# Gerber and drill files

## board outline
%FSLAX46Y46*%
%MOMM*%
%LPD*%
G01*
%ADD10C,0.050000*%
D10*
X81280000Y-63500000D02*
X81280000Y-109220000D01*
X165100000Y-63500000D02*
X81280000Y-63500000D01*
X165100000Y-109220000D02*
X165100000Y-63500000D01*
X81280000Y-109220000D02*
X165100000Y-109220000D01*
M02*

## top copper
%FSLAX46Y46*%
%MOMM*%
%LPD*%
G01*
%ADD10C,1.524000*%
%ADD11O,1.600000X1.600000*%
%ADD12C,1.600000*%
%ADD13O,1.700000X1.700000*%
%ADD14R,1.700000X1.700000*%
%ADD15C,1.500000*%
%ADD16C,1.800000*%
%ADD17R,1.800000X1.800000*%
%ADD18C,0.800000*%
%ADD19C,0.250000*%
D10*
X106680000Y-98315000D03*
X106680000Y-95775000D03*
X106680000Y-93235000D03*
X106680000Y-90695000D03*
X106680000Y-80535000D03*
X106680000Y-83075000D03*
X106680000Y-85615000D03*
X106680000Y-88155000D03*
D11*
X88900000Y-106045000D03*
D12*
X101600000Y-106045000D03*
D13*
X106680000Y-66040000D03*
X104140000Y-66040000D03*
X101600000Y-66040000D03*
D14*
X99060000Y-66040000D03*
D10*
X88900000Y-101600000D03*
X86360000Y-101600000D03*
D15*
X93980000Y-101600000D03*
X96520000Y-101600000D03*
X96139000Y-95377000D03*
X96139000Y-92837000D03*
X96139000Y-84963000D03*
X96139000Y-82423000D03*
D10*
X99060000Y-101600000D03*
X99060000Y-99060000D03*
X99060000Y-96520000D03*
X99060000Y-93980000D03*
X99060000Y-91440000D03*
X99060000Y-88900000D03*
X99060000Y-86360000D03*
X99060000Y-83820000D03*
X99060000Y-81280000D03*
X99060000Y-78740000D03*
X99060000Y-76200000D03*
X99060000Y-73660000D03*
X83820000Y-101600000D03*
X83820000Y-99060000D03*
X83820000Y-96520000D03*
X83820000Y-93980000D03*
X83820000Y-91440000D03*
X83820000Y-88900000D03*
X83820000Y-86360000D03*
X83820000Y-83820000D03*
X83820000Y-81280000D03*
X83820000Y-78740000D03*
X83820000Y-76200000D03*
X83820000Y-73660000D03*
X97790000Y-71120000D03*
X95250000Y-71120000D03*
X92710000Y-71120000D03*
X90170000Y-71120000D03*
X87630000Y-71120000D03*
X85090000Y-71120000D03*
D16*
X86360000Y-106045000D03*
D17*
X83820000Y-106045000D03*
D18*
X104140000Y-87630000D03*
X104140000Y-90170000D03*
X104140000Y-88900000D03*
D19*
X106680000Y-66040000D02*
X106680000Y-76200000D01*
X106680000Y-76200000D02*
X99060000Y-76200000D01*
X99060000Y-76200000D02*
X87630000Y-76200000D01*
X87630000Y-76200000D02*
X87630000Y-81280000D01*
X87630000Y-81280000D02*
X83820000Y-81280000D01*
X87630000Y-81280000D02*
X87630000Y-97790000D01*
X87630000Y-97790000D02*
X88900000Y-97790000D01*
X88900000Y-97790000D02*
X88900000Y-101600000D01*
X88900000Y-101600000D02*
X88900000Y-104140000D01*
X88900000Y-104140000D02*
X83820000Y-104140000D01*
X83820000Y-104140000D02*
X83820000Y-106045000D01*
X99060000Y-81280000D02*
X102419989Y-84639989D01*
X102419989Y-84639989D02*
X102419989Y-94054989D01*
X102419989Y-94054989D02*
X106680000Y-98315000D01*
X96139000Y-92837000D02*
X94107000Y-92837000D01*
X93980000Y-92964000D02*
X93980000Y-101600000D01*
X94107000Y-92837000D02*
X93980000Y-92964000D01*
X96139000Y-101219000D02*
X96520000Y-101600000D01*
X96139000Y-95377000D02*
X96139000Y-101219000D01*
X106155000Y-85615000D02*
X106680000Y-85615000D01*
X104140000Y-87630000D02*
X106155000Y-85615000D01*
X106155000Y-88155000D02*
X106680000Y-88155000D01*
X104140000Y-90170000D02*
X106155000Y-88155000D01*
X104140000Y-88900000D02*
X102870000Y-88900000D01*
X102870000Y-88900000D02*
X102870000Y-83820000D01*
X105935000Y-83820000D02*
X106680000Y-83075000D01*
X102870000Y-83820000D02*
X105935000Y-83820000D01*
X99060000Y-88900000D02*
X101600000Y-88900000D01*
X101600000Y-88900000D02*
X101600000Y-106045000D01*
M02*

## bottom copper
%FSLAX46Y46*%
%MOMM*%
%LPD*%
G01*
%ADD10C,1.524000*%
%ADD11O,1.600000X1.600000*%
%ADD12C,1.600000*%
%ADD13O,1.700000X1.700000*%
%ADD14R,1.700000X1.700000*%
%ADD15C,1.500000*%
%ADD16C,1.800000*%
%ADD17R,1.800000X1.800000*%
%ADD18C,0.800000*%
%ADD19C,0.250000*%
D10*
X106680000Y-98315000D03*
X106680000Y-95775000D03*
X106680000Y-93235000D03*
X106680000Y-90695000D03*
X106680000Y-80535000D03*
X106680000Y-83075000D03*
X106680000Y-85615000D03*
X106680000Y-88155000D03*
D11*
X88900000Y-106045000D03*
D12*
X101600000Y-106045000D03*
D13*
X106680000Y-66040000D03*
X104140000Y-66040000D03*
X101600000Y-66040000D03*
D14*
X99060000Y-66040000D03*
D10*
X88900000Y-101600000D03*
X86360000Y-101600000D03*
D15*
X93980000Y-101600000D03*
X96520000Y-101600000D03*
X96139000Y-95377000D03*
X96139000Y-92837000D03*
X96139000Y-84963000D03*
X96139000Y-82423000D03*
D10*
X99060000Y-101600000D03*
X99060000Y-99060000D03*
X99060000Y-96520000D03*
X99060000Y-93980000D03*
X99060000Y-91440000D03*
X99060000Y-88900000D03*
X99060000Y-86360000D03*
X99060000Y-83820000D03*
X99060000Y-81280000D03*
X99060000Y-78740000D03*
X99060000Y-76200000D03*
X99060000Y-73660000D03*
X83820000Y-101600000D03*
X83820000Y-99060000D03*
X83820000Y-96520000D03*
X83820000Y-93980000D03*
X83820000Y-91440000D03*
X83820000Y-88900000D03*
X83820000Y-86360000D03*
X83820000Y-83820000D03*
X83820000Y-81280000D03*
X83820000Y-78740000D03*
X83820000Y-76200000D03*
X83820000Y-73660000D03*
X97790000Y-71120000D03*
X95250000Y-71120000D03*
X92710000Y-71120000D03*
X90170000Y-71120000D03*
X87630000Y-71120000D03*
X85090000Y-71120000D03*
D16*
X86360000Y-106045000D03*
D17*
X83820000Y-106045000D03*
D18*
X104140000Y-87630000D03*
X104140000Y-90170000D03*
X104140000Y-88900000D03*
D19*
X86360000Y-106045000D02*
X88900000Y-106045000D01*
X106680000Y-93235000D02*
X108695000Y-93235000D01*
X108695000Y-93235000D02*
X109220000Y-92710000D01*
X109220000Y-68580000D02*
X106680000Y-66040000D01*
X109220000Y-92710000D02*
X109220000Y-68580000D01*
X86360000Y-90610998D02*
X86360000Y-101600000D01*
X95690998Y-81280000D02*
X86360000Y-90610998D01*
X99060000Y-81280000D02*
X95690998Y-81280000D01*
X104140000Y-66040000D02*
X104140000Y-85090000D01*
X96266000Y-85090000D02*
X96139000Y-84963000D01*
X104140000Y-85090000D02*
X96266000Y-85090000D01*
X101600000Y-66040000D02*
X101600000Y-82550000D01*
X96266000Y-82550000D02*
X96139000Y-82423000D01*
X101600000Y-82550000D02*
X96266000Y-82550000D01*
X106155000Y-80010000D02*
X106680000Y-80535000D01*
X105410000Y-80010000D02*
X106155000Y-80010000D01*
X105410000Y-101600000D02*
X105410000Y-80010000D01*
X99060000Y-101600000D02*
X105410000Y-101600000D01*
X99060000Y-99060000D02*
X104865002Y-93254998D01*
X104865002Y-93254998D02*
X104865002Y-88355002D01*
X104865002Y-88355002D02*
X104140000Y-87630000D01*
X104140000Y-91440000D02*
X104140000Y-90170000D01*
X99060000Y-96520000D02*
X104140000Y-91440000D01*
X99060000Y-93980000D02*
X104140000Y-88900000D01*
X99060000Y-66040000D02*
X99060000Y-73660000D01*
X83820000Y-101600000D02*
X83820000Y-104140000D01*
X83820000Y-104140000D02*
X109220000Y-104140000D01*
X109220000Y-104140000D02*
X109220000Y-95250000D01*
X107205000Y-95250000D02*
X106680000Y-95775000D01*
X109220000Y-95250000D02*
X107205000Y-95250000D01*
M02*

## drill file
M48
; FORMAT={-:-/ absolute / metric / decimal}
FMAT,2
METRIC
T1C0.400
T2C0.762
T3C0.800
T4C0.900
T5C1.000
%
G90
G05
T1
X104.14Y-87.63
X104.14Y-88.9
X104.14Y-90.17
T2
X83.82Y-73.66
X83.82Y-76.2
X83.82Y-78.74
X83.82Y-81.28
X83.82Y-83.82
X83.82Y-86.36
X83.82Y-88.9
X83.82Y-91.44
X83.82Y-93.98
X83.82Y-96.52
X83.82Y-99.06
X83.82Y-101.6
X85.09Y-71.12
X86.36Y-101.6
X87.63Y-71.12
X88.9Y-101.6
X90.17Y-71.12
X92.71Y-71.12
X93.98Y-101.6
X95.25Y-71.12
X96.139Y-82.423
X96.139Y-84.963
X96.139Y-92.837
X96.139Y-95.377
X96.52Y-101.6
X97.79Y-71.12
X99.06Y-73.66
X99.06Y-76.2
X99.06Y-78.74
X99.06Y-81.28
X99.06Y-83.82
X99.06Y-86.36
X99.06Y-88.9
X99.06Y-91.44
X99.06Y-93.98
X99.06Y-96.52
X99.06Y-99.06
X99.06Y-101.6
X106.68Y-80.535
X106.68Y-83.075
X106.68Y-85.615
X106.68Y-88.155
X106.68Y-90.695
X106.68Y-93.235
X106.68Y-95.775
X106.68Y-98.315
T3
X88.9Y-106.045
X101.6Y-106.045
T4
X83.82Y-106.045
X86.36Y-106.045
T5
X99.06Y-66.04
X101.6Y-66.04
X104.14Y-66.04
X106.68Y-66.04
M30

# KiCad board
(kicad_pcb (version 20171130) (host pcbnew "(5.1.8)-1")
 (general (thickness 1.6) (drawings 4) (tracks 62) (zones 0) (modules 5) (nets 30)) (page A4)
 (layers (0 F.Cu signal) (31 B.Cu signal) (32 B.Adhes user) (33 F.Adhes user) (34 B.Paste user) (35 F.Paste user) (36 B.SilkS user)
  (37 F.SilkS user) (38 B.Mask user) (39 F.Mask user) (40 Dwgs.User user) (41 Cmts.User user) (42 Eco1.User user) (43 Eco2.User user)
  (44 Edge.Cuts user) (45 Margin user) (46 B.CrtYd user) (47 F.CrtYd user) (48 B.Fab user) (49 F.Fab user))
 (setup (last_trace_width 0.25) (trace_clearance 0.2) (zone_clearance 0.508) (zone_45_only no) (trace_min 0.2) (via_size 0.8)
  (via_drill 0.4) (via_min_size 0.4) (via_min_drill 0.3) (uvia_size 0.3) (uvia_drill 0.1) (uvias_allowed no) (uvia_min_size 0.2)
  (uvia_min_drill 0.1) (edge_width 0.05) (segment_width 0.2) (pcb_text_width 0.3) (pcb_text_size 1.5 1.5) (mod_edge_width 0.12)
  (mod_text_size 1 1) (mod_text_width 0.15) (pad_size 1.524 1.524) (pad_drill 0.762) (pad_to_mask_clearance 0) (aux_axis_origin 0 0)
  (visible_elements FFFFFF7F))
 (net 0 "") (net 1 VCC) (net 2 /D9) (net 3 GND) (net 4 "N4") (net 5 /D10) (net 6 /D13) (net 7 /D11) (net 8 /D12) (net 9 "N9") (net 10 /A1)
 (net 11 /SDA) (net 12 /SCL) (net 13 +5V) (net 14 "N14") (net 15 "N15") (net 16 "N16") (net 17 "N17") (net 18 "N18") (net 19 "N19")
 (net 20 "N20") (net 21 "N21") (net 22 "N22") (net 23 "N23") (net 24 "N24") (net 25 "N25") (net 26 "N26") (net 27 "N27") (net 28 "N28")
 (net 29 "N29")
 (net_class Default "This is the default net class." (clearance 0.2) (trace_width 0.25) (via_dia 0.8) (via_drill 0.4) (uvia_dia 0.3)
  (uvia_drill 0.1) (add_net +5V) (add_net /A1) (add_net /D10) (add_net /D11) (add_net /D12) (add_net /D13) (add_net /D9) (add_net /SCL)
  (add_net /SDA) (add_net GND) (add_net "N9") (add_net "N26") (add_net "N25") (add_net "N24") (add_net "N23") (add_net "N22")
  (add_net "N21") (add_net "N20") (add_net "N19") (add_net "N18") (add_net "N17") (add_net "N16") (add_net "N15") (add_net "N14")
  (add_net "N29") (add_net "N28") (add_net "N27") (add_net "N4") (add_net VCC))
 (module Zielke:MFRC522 (layer F.Cu) (at 106.68 88.155)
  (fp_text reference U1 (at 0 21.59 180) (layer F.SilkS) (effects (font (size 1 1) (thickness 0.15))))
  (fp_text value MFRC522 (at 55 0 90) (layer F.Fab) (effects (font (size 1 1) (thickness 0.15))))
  (pad 8 thru_hole circle (at 0 10.16) (size 1.524 1.524) (drill 0.762) (layers *.Cu *.Mask) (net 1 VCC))
  (pad 7 thru_hole circle (at 0 7.62) (size 1.524 1.524) (drill 0.762) (layers *.Cu *.Mask) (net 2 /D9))
  (pad 6 thru_hole circle (at 0 5.08) (size 1.524 1.524) (drill 0.762) (layers *.Cu *.Mask) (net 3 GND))
  (pad 5 thru_hole circle (at 0 2.54) (size 1.524 1.524) (drill 0.762) (layers *.Cu *.Mask) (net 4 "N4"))
  (pad 1 thru_hole circle (at 0 -7.62) (size 1.524 1.524) (drill 0.762) (layers *.Cu *.Mask) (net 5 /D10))
  (pad 2 thru_hole circle (at 0 -5.08) (size 1.524 1.524) (drill 0.762) (layers *.Cu *.Mask) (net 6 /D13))
  (pad 3 thru_hole circle (at 0 -2.54) (size 1.524 1.524) (drill 0.762) (layers *.Cu *.Mask) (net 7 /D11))
  (pad 4 thru_hole circle (at 0 0) (size 1.524 1.524) (drill 0.762) (layers *.Cu *.Mask) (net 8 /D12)))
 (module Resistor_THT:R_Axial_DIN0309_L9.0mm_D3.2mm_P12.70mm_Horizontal (layer F.Cu) (at 101.6 106.045 180)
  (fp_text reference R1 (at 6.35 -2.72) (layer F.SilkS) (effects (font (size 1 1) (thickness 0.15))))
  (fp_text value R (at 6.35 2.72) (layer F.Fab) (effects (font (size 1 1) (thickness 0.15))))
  (pad 2 thru_hole oval (at 12.7 0 180) (size 1.6 1.6) (drill 0.8) (layers *.Cu *.Mask) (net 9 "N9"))
  (pad 1 thru_hole circle (at 0 0 180) (size 1.6 1.6) (drill 0.8) (layers *.Cu *.Mask) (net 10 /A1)))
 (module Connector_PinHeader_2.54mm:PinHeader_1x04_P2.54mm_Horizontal (layer F.Cu) (at 99.06 66.04 90)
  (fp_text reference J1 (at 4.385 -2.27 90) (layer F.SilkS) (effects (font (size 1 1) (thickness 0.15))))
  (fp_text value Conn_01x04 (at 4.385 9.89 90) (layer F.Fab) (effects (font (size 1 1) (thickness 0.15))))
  (pad 4 thru_hole oval (at 0 7.62 90) (size 1.7 1.7) (drill 1) (layers *.Cu *.Mask) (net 3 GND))
  (pad 3 thru_hole oval (at 0 5.08 90) (size 1.7 1.7) (drill 1) (layers *.Cu *.Mask) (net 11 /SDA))
  (pad 2 thru_hole oval (at 0 2.54 90) (size 1.7 1.7) (drill 1) (layers *.Cu *.Mask) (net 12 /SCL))
  (pad 1 thru_hole rect (at 0 0 90) (size 1.7 1.7) (drill 1) (layers *.Cu *.Mask) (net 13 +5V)))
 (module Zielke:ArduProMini (layer F.Cu) (at 91.44 86.36)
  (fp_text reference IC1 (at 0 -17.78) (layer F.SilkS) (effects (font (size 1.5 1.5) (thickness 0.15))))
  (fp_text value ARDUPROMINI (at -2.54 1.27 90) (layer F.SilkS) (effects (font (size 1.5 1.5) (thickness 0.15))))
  (pad 20 thru_hole circle (at -2.54 15.24) (size 1.524 1.524) (drill 0.762) (layers *.Cu *.Mask) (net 3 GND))
  (pad 22 thru_hole circle (at -5.08 15.24) (size 1.524 1.524) (drill 0.762) (layers *.Cu *.Mask) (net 1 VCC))
  (pad 34 thru_hole circle (at 2.54 15.24) (size 1.5 1.5) (drill 0.762) (layers *.Cu *.Mask) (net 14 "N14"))
  (pad 33 thru_hole circle (at 5.08 15.24) (size 1.5 1.5) (drill 0.762) (layers *.Cu *.Mask) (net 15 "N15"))
  (pad 33 thru_hole circle (at 4.699 9.017) (size 1.5 1.5) (drill 0.762) (layers *.Cu *.Mask) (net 15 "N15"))
  (pad 34 thru_hole circle (at 4.699 6.477) (size 1.5 1.5) (drill 0.762) (layers *.Cu *.Mask) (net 14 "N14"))
  (pad 31 thru_hole circle (at 4.699 -1.397) (size 1.5 1.5) (drill 0.762) (layers *.Cu *.Mask) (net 11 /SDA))
  (pad 32 thru_hole circle (at 4.699 -3.937) (size 1.5 1.5) (drill 0.762) (layers *.Cu *.Mask) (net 12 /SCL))
  (pad 30 thru_hole circle (at 7.62 15.24) (size 1.524 1.524) (drill 0.762) (layers *.Cu *.Mask) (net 5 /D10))
  (pad 29 thru_hole circle (at 7.62 12.7) (size 1.524 1.524) (drill 0.762) (layers *.Cu *.Mask) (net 7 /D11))
  (pad 28 thru_hole circle (at 7.62 10.16) (size 1.524 1.524) (drill 0.762) (layers *.Cu *.Mask) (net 8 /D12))
  (pad 27 thru_hole circle (at 7.62 7.62) (size 1.524 1.524) (drill 0.762) (layers *.Cu *.Mask) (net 6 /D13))
  (pad 26 thru_hole circle (at 7.62 5.08) (size 1.524 1.524) (drill 0.762) (layers *.Cu *.Mask) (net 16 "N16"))
  (pad 25 thru_hole circle (at 7.62 2.54) (size 1.524 1.524) (drill 0.762) (layers *.Cu *.Mask) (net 10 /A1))
  (pad 24 thru_hole circle (at 7.62 0) (size 1.524 1.524) (drill 0.762) (layers *.Cu *.Mask) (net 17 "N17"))
  (pad 23 thru_hole circle (at 7.62 -2.54) (size 1.524 1.524) (drill 0.762) (layers *.Cu *.Mask) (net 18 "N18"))
  (pad 22 thru_hole circle (at 7.62 -5.08) (size 1.524 1.524) (drill 0.762) (layers *.Cu *.Mask) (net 1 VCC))
  (pad 21 thru_hole circle (at 7.62 -7.62) (size 1.524 1.524) (drill 0.762) (layers *.Cu *.Mask) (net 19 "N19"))
  (pad 20 thru_hole circle (at 7.62 -10.16) (size 1.524 1.524) (drill 0.762) (layers *.Cu *.Mask) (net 3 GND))
  (pad 19 thru_hole circle (at 7.62 -12.7) (size 1.524 1.524) (drill 0.762) (layers *.Cu *.Mask) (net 13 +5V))
  (pad 18 thru_hole circle (at -7.62 15.24) (size 1.524 1.524) (drill 0.762) (layers *.Cu *.Mask) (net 2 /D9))
  (pad 17 thru_hole circle (at -7.62 12.7) (size 1.524 1.524) (drill 0.762) (layers *.Cu *.Mask) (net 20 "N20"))
  (pad 16 thru_hole circle (at -7.62 10.16) (size 1.524 1.524) (drill 0.762) (layers *.Cu *.Mask) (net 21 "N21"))
  (pad 15 thru_hole circle (at -7.62 7.62) (size 1.524 1.524) (drill 0.762) (layers *.Cu *.Mask) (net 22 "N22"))
  (pad 14 thru_hole circle (at -7.62 5.08) (size 1.524 1.524) (drill 0.762) (layers *.Cu *.Mask) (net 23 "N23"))
  (pad 13 thru_hole circle (at -7.62 2.54) (size 1.524 1.524) (drill 0.762) (layers *.Cu *.Mask) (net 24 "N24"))
  (pad 12 thru_hole circle (at -7.62 0) (size 1.524 1.524) (drill 0.762) (layers *.Cu *.Mask) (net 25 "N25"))
  (pad 11 thru_hole circle (at -7.62 -2.54) (size 1.524 1.524) (drill 0.762) (layers *.Cu *.Mask) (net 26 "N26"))
  (pad 10 thru_hole circle (at -7.62 -5.08) (size 1.524 1.524) (drill 0.762) (layers *.Cu *.Mask) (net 3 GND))
  (pad 9 thru_hole circle (at -7.62 -7.62) (size 1.524 1.524) (drill 0.762) (layers *.Cu *.Mask) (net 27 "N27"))
  (pad 8 thru_hole circle (at -7.62 -10.16) (size 1.524 1.524) (drill 0.762) (layers *.Cu *.Mask) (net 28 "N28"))
  (pad 7 thru_hole circle (at -7.62 -12.7) (size 1.524 1.524) (drill 0.762) (layers *.Cu *.Mask) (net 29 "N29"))
  (pad 1 thru_hole circle (at 6.35 -15.24) (size 1.524 1.524) (drill 0.762) (layers *.Cu *.Mask))
  (pad 2 thru_hole circle (at 3.81 -15.24) (size 1.524 1.524) (drill 0.762) (layers *.Cu *.Mask))
  (pad 3 thru_hole circle (at 1.27 -15.24) (size 1.524 1.524) (drill 0.762) (layers *.Cu *.Mask))
  (pad 4 thru_hole circle (at -1.27 -15.24) (size 1.524 1.524) (drill 0.762) (layers *.Cu *.Mask))
  (pad 5 thru_hole circle (at -3.81 -15.24) (size 1.524 1.524) (drill 0.762) (layers *.Cu *.Mask))
  (pad 6 thru_hole circle (at -6.35 -15.24) (size 1.524 1.524) (drill 0.762) (layers *.Cu *.Mask)))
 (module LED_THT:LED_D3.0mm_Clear (layer F.Cu) (at 83.82 106.045)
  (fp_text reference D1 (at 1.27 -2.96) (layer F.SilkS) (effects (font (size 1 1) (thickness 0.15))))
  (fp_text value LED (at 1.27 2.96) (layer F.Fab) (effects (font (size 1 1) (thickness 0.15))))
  (pad 2 thru_hole circle (at 2.54 0) (size 1.8 1.8) (drill 0.9) (layers *.Cu *.Mask) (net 9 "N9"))
  (pad 1 thru_hole rect (at 0 0) (size 1.8 1.8) (drill 0.9) (layers *.Cu *.Mask) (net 3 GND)))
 (gr_line (start 81.28 63.5) (end 81.28 109.22) (layer Edge.Cuts) (width 0.05))
 (gr_line (start 165.1 63.5) (end 81.28 63.5) (layer Edge.Cuts) (width 0.05))
 (gr_line (start 165.1 109.22) (end 165.1 63.5) (layer Edge.Cuts) (width 0.05))
 (gr_line (start 81.28 109.22) (end 165.1 109.22) (layer Edge.Cuts) (width 0.05))
 (segment (start 86.36 106.045) (end 88.9 106.045) (width 0.25) (layer B.Cu) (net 9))
 (segment (start 106.68 66.04) (end 106.68 76.2) (width 0.25) (layer F.Cu) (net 3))
 (segment (start 106.68 76.2) (end 99.06 76.2) (width 0.25) (layer F.Cu) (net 3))
 (segment (start 99.06 76.2) (end 87.63 76.2) (width 0.25) (layer F.Cu) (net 3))
 (segment (start 87.63 76.2) (end 87.63 81.28) (width 0.25) (layer F.Cu) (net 3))
 (segment (start 87.63 81.28) (end 83.82 81.28) (width 0.25) (layer F.Cu) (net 3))
 (segment (start 87.63 81.28) (end 87.63 97.79) (width 0.25) (layer F.Cu) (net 3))
 (segment (start 87.63 97.79) (end 88.9 97.79) (width 0.25) (layer F.Cu) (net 3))
 (segment (start 88.9 97.79) (end 88.9 101.6) (width 0.25) (layer F.Cu) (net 3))
 (segment (start 88.9 101.6) (end 88.9 104.14) (width 0.25) (layer F.Cu) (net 3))
 (segment (start 88.9 104.14) (end 83.82 104.14) (width 0.25) (layer F.Cu) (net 3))
 (segment (start 83.82 104.14) (end 83.82 106.045) (width 0.25) (layer F.Cu) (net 3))
 (segment (start 106.68 93.235) (end 108.695 93.235) (width 0.25) (layer B.Cu) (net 3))
 (segment (start 108.695 93.235) (end 109.22 92.71) (width 0.25) (layer B.Cu) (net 3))
 (segment (start 109.22 68.58) (end 106.68 66.04) (width 0.25) (layer B.Cu) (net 3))
 (segment (start 109.22 92.71) (end 109.22 68.58) (width 0.25) (layer B.Cu) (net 3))
 (segment (start 86.36 90.610998) (end 86.36 101.6) (width 0.25) (layer B.Cu) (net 1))
 (segment (start 95.690998 81.28) (end 86.36 90.610998) (width 0.25) (layer B.Cu) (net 1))
 (segment (start 99.06 81.28) (end 95.690998 81.28) (width 0.25) (layer B.Cu) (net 1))
 (segment (start 99.06 81.28) (end 102.419989 84.639989) (width 0.25) (layer F.Cu) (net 1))
 (segment (start 102.419989 84.639989) (end 102.419989 94.054989) (width 0.25) (layer F.Cu) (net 1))
 (segment (start 102.419989 94.054989) (end 106.68 98.315) (width 0.25) (layer F.Cu) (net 1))
 (segment (start 96.139 92.837) (end 94.107 92.837) (width 0.25) (layer F.Cu) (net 14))
 (segment (start 93.98 92.964) (end 93.98 101.6) (width 0.25) (layer F.Cu) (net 14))
 (segment (start 94.107 92.837) (end 93.98 92.964) (width 0.25) (layer F.Cu) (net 14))
 (segment (start 96.139 101.219) (end 96.52 101.6) (width 0.25) (layer F.Cu) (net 15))
 (segment (start 96.139 95.377) (end 96.139 101.219) (width 0.25) (layer F.Cu) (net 15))
 (segment (start 104.14 66.04) (end 104.14 85.09) (width 0.25) (layer B.Cu) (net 11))
 (segment (start 96.266 85.09) (end 96.139 84.963) (width 0.25) (layer B.Cu) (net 11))
 (segment (start 104.14 85.09) (end 96.266 85.09) (width 0.25) (layer B.Cu) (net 11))
 (segment (start 101.6 66.04) (end 101.6 82.55) (width 0.25) (layer B.Cu) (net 12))
 (segment (start 96.266 82.55) (end 96.139 82.423) (width 0.25) (layer B.Cu) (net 12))
 (segment (start 101.6 82.55) (end 96.266 82.55) (width 0.25) (layer B.Cu) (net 12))
 (segment (start 106.155 80.01) (end 106.68 80.535) (width 0.25) (layer B.Cu) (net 5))
 (segment (start 105.41 80.01) (end 106.155 80.01) (width 0.25) (layer B.Cu) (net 5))
 (segment (start 105.41 101.6) (end 105.41 80.01) (width 0.25) (layer B.Cu) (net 5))
 (segment (start 99.06 101.6) (end 105.41 101.6) (width 0.25) (layer B.Cu) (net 5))
 (via (at 104.14 87.63) (size 0.8) (drill 0.4) (layers F.Cu B.Cu) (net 7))
 (segment (start 106.155 85.615) (end 106.68 85.615) (width 0.25) (layer F.Cu) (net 7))
 (segment (start 104.14 87.63) (end 106.155 85.615) (width 0.25) (layer F.Cu) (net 7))
 (segment (start 99.06 99.06) (end 104.865002 93.254998) (width 0.25) (layer B.Cu) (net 7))
 (segment (start 104.865002 93.254998) (end 104.865002 88.355002) (width 0.25) (layer B.Cu) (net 7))
 (segment (start 104.865002 88.355002) (end 104.14 87.63) (width 0.25) (layer B.Cu) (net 7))
 (via (at 104.14 90.17) (size 0.8) (drill 0.4) (layers F.Cu B.Cu) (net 8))
 (segment (start 104.14 91.44) (end 104.14 90.17) (width 0.25) (layer B.Cu) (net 8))
 (segment (start 99.06 96.52) (end 104.14 91.44) (width 0.25) (layer B.Cu) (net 8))
 (segment (start 106.155 88.155) (end 106.68 88.155) (width 0.25) (layer F.Cu) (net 8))
 (segment (start 104.14 90.17) (end 106.155 88.155) (width 0.25) (layer F.Cu) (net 8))
 (via (at 104.14 88.9) (size 0.8) (drill 0.4) (layers F.Cu B.Cu) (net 6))
 (segment (start 99.06 93.98) (end 104.14 88.9) (width 0.25) (layer B.Cu) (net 6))
 (segment (start 104.14 88.9) (end 102.87 88.9) (width 0.25) (layer F.Cu) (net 6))
 (segment (start 102.87 88.9) (end 102.87 83.82) (width 0.25) (layer F.Cu) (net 6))
 (segment (start 105.935 83.82) (end 106.68 83.075) (width 0.25) (layer F.Cu) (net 6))
 (segment (start 102.87 83.82) (end 105.935 83.82) (width 0.25) (layer F.Cu) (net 6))
 (segment (start 99.06 88.9) (end 101.6 88.9) (width 0.25) (layer F.Cu) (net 10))
 (segment (start 101.6 88.9) (end 101.6 106.045) (width 0.25) (layer F.Cu) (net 10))
 (segment (start 99.06 66.04) (end 99.06 73.66) (width 0.25) (layer B.Cu) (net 13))
 (segment (start 83.82 101.6) (end 83.82 104.14) (width 0.25) (layer B.Cu) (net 2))
 (segment (start 83.82 104.14) (end 109.22 104.14) (width 0.25) (layer B.Cu) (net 2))
 (segment (start 109.22 104.14) (end 109.22 95.25) (width 0.25) (layer B.Cu) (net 2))
 (segment (start 107.205 95.25) (end 106.68 95.775) (width 0.25) (layer B.Cu) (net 2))
 (segment (start 109.22 95.25) (end 107.205 95.25) (width 0.25) (layer B.Cu) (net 2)))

